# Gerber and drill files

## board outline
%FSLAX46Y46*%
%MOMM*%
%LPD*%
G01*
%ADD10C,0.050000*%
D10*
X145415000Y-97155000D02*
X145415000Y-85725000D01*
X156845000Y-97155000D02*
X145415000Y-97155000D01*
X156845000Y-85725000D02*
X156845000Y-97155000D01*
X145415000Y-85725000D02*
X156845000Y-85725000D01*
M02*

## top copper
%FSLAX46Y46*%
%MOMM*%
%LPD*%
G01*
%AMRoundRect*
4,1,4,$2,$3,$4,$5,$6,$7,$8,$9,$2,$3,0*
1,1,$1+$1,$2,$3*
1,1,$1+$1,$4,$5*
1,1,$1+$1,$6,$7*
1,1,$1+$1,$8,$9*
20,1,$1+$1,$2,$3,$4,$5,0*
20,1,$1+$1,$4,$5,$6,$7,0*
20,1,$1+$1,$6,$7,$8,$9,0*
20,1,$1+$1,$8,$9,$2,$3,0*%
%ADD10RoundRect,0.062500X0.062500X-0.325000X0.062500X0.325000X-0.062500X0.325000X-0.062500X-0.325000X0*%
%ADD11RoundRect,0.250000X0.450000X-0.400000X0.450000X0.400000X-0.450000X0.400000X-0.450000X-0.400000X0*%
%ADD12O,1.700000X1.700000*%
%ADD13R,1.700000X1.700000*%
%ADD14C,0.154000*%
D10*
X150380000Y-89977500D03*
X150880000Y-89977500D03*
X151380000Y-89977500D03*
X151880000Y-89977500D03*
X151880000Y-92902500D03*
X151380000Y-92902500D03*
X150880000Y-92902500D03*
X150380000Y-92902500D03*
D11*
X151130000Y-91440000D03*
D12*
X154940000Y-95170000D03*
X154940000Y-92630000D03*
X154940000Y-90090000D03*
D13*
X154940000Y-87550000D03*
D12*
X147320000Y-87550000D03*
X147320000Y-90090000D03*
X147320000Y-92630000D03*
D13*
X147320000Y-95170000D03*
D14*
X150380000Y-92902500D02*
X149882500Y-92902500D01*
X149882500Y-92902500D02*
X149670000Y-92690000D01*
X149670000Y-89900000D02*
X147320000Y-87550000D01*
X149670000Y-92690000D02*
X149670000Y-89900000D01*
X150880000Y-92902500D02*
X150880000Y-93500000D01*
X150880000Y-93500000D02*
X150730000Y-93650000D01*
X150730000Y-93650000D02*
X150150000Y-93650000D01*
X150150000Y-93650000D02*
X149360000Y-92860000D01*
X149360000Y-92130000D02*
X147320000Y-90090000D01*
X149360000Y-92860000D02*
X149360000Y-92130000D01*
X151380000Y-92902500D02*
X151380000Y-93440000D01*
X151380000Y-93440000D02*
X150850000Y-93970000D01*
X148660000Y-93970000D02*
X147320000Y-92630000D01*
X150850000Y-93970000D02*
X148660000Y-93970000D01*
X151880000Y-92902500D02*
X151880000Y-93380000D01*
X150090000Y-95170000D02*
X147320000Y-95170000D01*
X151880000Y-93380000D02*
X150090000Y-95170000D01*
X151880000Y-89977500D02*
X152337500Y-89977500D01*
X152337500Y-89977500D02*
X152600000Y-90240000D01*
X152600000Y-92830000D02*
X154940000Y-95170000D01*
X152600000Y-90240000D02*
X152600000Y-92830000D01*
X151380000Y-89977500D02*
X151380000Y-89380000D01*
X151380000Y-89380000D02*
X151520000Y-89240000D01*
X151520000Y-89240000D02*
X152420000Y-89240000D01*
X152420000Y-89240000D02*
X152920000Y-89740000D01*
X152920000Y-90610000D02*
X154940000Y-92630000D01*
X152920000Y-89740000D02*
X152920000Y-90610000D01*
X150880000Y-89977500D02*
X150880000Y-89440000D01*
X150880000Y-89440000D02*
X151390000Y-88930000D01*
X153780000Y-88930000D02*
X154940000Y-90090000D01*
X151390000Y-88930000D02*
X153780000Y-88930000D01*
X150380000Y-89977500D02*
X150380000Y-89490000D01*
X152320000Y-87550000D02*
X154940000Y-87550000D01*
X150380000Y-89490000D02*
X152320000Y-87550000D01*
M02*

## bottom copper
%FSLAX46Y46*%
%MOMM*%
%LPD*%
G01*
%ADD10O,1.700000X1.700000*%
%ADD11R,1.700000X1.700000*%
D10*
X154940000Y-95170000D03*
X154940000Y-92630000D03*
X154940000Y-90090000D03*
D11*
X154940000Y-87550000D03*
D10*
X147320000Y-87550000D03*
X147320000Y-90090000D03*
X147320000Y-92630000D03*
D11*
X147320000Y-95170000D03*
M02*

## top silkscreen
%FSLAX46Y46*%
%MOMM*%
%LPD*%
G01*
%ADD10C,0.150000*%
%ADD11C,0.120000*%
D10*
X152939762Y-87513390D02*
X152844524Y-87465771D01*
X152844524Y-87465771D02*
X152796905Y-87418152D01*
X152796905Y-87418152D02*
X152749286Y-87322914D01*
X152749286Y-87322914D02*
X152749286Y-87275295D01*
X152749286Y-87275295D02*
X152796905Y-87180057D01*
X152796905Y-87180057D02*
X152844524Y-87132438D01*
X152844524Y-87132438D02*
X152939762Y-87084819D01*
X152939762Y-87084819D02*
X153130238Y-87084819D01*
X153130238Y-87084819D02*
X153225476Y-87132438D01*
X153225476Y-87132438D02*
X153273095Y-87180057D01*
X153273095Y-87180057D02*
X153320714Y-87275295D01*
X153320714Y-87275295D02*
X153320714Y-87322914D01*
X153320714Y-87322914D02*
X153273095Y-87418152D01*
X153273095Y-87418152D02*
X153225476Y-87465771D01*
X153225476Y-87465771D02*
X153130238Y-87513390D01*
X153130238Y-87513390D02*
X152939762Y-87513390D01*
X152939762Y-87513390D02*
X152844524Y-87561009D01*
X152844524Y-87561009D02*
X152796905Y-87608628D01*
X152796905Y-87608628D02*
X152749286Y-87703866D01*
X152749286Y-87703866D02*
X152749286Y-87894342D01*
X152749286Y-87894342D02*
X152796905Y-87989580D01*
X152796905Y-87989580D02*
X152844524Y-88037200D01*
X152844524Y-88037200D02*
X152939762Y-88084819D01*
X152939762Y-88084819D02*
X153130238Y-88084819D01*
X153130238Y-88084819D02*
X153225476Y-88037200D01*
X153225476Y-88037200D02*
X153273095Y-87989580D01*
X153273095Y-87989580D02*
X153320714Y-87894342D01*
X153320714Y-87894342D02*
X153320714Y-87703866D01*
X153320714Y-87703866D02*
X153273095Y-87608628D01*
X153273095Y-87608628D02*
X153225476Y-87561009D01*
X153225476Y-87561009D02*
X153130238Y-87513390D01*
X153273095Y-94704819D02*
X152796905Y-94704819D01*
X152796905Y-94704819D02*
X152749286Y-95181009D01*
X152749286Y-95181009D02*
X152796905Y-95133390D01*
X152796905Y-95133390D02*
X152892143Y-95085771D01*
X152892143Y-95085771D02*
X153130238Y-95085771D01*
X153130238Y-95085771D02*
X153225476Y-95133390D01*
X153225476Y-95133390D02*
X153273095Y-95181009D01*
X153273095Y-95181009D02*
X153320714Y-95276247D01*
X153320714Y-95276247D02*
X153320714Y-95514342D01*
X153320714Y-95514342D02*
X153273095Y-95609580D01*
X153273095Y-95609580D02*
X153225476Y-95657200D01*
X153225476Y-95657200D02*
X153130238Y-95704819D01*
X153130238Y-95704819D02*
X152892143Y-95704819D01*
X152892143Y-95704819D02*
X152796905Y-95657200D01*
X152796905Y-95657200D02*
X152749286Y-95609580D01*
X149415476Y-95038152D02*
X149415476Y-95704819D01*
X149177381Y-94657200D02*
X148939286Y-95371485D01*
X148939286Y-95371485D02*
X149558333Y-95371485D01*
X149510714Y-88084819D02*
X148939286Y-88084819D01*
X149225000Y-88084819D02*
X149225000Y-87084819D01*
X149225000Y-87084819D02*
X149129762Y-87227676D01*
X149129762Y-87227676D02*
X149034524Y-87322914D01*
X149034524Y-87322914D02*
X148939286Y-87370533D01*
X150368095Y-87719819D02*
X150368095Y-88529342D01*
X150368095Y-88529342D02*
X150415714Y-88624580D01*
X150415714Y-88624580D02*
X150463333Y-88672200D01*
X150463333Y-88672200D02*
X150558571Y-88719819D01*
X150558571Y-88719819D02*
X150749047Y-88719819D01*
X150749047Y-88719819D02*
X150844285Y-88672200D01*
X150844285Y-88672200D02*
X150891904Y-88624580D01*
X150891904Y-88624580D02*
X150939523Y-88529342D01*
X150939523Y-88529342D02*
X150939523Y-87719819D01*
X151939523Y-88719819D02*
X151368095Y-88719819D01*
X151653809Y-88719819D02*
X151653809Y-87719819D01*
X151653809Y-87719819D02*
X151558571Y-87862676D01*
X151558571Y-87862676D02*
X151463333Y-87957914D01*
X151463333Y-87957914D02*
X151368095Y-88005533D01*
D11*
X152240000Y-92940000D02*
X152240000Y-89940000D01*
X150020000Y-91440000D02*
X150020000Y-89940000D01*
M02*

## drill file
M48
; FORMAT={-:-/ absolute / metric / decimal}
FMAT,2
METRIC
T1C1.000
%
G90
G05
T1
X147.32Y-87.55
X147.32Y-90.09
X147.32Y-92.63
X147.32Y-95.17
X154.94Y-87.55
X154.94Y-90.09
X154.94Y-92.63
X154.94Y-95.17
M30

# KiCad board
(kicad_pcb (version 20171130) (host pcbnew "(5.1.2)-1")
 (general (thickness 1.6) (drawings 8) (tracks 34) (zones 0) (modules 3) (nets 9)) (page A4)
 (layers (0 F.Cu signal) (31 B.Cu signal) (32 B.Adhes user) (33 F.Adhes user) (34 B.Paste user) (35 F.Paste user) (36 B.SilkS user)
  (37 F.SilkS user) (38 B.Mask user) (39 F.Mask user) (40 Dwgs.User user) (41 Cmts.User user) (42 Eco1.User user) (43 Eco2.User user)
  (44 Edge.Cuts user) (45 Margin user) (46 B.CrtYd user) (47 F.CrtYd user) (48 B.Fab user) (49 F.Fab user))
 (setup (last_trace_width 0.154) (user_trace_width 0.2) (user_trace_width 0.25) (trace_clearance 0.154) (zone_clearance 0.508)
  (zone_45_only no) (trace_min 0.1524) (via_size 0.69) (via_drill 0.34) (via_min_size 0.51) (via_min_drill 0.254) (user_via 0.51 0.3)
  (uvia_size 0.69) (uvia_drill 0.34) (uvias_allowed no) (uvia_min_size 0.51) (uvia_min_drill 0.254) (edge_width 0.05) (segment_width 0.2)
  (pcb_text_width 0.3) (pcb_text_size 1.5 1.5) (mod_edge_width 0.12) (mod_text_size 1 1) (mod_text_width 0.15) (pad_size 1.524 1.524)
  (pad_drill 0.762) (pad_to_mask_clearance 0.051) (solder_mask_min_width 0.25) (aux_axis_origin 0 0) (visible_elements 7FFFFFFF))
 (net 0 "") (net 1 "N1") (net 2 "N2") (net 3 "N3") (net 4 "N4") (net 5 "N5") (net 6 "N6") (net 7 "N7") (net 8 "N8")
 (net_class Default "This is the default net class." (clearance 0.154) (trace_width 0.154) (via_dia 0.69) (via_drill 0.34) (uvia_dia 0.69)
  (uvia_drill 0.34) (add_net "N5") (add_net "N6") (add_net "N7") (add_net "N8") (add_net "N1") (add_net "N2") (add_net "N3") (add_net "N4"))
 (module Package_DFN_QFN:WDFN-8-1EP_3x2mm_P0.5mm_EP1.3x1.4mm (layer F.Cu) (at 151.13 91.44 90)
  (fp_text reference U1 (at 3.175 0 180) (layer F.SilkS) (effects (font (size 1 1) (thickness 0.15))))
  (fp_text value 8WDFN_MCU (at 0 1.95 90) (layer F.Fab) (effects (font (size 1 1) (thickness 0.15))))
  (fp_line (start -1.5 1.11) (end 1.5 1.11) (layer F.SilkS) (width 0.12))
  (fp_line (start 0 -1.11) (end 1.5 -1.11) (layer F.SilkS) (width 0.12))
  (pad 8 smd roundrect (at 1.4625 -0.75 90) (size 0.775 0.25) (layers F.Cu F.Paste F.Mask) (roundrect_rratio 0.25) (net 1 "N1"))
  (pad 7 smd roundrect (at 1.4625 -0.25 90) (size 0.775 0.25) (layers F.Cu F.Paste F.Mask) (roundrect_rratio 0.25) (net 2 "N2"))
  (pad 6 smd roundrect (at 1.4625 0.25 90) (size 0.775 0.25) (layers F.Cu F.Paste F.Mask) (roundrect_rratio 0.25) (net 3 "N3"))
  (pad 5 smd roundrect (at 1.4625 0.75 90) (size 0.775 0.25) (layers F.Cu F.Paste F.Mask) (roundrect_rratio 0.25) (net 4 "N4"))
  (pad 4 smd roundrect (at -1.4625 0.75 90) (size 0.775 0.25) (layers F.Cu F.Paste F.Mask) (roundrect_rratio 0.25) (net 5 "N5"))
  (pad 3 smd roundrect (at -1.4625 0.25 90) (size 0.775 0.25) (layers F.Cu F.Paste F.Mask) (roundrect_rratio 0.25) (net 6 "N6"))
  (pad 2 smd roundrect (at -1.4625 -0.25 90) (size 0.775 0.25) (layers F.Cu F.Paste F.Mask) (roundrect_rratio 0.25) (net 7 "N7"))
  (pad 1 smd roundrect (at -1.4625 -0.75 90) (size 0.775 0.25) (layers F.Cu F.Paste F.Mask) (roundrect_rratio 0.25) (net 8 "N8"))
  (pad "" smd roundrect (at 0.325 0.35 90) (size 0.52 0.56) (layers F.Paste) (roundrect_rratio 0.25))
  (pad "" smd roundrect (at 0.325 -0.35 90) (size 0.52 0.56) (layers F.Paste) (roundrect_rratio 0.25))
  (pad "" smd roundrect (at -0.325 0.35 90) (size 0.52 0.56) (layers F.Paste) (roundrect_rratio 0.25))
  (pad "" smd roundrect (at -0.325 -0.35 90) (size 0.52 0.56) (layers F.Paste) (roundrect_rratio 0.25))
  (pad 9 smd roundrect (at 0 0 90) (size 1.3 1.4) (layers F.Cu F.Mask) (roundrect_rratio 0.192308)))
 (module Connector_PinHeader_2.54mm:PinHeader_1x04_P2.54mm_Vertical (layer B.Cu) (at 154.94 87.55 180)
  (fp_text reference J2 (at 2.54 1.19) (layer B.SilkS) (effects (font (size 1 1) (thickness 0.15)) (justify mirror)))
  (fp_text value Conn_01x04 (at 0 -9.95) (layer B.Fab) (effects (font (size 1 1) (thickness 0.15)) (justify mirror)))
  (pad 4 thru_hole oval (at 0 -7.62 180) (size 1.7 1.7) (drill 1) (layers *.Cu *.Mask) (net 4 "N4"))
  (pad 3 thru_hole oval (at 0 -5.08 180) (size 1.7 1.7) (drill 1) (layers *.Cu *.Mask) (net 3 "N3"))
  (pad 2 thru_hole oval (at 0 -2.54 180) (size 1.7 1.7) (drill 1) (layers *.Cu *.Mask) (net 2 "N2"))
  (pad 1 thru_hole rect (at 0 0 180) (size 1.7 1.7) (drill 1) (layers *.Cu *.Mask) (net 1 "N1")))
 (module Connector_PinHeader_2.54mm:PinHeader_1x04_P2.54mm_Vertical (layer B.Cu) (at 147.32 95.17)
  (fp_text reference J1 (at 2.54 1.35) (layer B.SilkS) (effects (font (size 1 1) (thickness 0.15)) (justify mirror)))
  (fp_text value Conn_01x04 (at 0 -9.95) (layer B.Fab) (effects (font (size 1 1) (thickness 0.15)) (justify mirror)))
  (pad 4 thru_hole oval (at 0 -7.62) (size 1.7 1.7) (drill 1) (layers *.Cu *.Mask) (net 8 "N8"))
  (pad 3 thru_hole oval (at 0 -5.08) (size 1.7 1.7) (drill 1) (layers *.Cu *.Mask) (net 7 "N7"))
  (pad 2 thru_hole oval (at 0 -2.54) (size 1.7 1.7) (drill 1) (layers *.Cu *.Mask) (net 6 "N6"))
  (pad 1 thru_hole rect (at 0 0) (size 1.7 1.7) (drill 1) (layers *.Cu *.Mask) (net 5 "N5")))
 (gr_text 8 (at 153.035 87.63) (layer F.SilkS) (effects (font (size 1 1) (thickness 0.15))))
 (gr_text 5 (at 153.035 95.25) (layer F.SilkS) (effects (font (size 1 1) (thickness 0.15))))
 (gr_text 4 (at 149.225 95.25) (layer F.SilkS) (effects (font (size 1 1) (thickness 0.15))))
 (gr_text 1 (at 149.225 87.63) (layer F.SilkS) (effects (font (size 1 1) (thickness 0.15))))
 (gr_line (start 145.415 97.155) (end 145.415 85.725) (layer Edge.Cuts) (width 0.05))
 (gr_line (start 156.845 97.155) (end 145.415 97.155) (layer Edge.Cuts) (width 0.05))
 (gr_line (start 156.845 85.725) (end 156.845 97.155) (layer Edge.Cuts) (width 0.05))
 (gr_line (start 145.415 85.725) (end 156.845 85.725) (layer Edge.Cuts) (width 0.05))
 (segment (start 150.38 92.9025) (end 149.8825 92.9025) (width 0.154) (layer F.Cu) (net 8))
 (segment (start 149.8825 92.9025) (end 149.67 92.69) (width 0.154) (layer F.Cu) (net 8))
 (segment (start 149.67 89.9) (end 147.32 87.55) (width 0.154) (layer F.Cu) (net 8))
 (segment (start 149.67 92.69) (end 149.67 89.9) (width 0.154) (layer F.Cu) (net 8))
 (segment (start 150.88 92.9025) (end 150.88 93.5) (width 0.154) (layer F.Cu) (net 7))
 (segment (start 150.88 93.5) (end 150.73 93.65) (width 0.154) (layer F.Cu) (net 7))
 (segment (start 150.73 93.65) (end 150.15 93.65) (width 0.154) (layer F.Cu) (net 7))
 (segment (start 150.15 93.65) (end 149.36 92.86) (width 0.154) (layer F.Cu) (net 7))
 (segment (start 149.36 92.13) (end 147.32 90.09) (width 0.154) (layer F.Cu) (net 7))
 (segment (start 149.36 92.86) (end 149.36 92.13) (width 0.154) (layer F.Cu) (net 7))
 (segment (start 151.38 92.9025) (end 151.38 93.44) (width 0.154) (layer F.Cu) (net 6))
 (segment (start 151.38 93.44) (end 150.85 93.97) (width 0.154) (layer F.Cu) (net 6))
 (segment (start 148.66 93.97) (end 147.32 92.63) (width 0.154) (layer F.Cu) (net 6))
 (segment (start 150.85 93.97) (end 148.66 93.97) (width 0.154) (layer F.Cu) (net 6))
 (segment (start 151.88 92.9025) (end 151.88 93.38) (width 0.154) (layer F.Cu) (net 5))
 (segment (start 150.09 95.17) (end 147.32 95.17) (width 0.154) (layer F.Cu) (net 5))
 (segment (start 151.88 93.38) (end 150.09 95.17) (width 0.154) (layer F.Cu) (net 5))
 (segment (start 151.88 89.9775) (end 152.3375 89.9775) (width 0.154) (layer F.Cu) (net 4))
 (segment (start 152.3375 89.9775) (end 152.6 90.24) (width 0.154) (layer F.Cu) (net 4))
 (segment (start 152.6 92.83) (end 154.94 95.17) (width 0.154) (layer F.Cu) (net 4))
 (segment (start 152.6 90.24) (end 152.6 92.83) (width 0.154) (layer F.Cu) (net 4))
 (segment (start 151.38 89.9775) (end 151.38 89.38) (width 0.154) (layer F.Cu) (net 3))
 (segment (start 151.38 89.38) (end 151.52 89.24) (width 0.154) (layer F.Cu) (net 3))
 (segment (start 151.52 89.24) (end 152.42 89.24) (width 0.154) (layer F.Cu) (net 3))
 (segment (start 152.42 89.24) (end 152.92 89.74) (width 0.154) (layer F.Cu) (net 3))
 (segment (start 152.92 90.61) (end 154.94 92.63) (width 0.154) (layer F.Cu) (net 3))
 (segment (start 152.92 89.74) (end 152.92 90.61) (width 0.154) (layer F.Cu) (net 3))
 (segment (start 150.88 89.9775) (end 150.88 89.44) (width 0.154) (layer F.Cu) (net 2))
 (segment (start 150.88 89.44) (end 151.39 88.93) (width 0.154) (layer F.Cu) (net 2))
 (segment (start 153.78 88.93) (end 154.94 90.09) (width 0.154) (layer F.Cu) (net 2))
 (segment (start 151.39 88.93) (end 153.78 88.93) (width 0.154) (layer F.Cu) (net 2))
 (segment (start 150.38 89.9775) (end 150.38 89.49) (width 0.154) (layer F.Cu) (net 1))
 (segment (start 152.32 87.55) (end 154.94 87.55) (width 0.154) (layer F.Cu) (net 1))
 (segment (start 150.38 89.49) (end 152.32 87.55) (width 0.154) (layer F.Cu) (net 1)))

